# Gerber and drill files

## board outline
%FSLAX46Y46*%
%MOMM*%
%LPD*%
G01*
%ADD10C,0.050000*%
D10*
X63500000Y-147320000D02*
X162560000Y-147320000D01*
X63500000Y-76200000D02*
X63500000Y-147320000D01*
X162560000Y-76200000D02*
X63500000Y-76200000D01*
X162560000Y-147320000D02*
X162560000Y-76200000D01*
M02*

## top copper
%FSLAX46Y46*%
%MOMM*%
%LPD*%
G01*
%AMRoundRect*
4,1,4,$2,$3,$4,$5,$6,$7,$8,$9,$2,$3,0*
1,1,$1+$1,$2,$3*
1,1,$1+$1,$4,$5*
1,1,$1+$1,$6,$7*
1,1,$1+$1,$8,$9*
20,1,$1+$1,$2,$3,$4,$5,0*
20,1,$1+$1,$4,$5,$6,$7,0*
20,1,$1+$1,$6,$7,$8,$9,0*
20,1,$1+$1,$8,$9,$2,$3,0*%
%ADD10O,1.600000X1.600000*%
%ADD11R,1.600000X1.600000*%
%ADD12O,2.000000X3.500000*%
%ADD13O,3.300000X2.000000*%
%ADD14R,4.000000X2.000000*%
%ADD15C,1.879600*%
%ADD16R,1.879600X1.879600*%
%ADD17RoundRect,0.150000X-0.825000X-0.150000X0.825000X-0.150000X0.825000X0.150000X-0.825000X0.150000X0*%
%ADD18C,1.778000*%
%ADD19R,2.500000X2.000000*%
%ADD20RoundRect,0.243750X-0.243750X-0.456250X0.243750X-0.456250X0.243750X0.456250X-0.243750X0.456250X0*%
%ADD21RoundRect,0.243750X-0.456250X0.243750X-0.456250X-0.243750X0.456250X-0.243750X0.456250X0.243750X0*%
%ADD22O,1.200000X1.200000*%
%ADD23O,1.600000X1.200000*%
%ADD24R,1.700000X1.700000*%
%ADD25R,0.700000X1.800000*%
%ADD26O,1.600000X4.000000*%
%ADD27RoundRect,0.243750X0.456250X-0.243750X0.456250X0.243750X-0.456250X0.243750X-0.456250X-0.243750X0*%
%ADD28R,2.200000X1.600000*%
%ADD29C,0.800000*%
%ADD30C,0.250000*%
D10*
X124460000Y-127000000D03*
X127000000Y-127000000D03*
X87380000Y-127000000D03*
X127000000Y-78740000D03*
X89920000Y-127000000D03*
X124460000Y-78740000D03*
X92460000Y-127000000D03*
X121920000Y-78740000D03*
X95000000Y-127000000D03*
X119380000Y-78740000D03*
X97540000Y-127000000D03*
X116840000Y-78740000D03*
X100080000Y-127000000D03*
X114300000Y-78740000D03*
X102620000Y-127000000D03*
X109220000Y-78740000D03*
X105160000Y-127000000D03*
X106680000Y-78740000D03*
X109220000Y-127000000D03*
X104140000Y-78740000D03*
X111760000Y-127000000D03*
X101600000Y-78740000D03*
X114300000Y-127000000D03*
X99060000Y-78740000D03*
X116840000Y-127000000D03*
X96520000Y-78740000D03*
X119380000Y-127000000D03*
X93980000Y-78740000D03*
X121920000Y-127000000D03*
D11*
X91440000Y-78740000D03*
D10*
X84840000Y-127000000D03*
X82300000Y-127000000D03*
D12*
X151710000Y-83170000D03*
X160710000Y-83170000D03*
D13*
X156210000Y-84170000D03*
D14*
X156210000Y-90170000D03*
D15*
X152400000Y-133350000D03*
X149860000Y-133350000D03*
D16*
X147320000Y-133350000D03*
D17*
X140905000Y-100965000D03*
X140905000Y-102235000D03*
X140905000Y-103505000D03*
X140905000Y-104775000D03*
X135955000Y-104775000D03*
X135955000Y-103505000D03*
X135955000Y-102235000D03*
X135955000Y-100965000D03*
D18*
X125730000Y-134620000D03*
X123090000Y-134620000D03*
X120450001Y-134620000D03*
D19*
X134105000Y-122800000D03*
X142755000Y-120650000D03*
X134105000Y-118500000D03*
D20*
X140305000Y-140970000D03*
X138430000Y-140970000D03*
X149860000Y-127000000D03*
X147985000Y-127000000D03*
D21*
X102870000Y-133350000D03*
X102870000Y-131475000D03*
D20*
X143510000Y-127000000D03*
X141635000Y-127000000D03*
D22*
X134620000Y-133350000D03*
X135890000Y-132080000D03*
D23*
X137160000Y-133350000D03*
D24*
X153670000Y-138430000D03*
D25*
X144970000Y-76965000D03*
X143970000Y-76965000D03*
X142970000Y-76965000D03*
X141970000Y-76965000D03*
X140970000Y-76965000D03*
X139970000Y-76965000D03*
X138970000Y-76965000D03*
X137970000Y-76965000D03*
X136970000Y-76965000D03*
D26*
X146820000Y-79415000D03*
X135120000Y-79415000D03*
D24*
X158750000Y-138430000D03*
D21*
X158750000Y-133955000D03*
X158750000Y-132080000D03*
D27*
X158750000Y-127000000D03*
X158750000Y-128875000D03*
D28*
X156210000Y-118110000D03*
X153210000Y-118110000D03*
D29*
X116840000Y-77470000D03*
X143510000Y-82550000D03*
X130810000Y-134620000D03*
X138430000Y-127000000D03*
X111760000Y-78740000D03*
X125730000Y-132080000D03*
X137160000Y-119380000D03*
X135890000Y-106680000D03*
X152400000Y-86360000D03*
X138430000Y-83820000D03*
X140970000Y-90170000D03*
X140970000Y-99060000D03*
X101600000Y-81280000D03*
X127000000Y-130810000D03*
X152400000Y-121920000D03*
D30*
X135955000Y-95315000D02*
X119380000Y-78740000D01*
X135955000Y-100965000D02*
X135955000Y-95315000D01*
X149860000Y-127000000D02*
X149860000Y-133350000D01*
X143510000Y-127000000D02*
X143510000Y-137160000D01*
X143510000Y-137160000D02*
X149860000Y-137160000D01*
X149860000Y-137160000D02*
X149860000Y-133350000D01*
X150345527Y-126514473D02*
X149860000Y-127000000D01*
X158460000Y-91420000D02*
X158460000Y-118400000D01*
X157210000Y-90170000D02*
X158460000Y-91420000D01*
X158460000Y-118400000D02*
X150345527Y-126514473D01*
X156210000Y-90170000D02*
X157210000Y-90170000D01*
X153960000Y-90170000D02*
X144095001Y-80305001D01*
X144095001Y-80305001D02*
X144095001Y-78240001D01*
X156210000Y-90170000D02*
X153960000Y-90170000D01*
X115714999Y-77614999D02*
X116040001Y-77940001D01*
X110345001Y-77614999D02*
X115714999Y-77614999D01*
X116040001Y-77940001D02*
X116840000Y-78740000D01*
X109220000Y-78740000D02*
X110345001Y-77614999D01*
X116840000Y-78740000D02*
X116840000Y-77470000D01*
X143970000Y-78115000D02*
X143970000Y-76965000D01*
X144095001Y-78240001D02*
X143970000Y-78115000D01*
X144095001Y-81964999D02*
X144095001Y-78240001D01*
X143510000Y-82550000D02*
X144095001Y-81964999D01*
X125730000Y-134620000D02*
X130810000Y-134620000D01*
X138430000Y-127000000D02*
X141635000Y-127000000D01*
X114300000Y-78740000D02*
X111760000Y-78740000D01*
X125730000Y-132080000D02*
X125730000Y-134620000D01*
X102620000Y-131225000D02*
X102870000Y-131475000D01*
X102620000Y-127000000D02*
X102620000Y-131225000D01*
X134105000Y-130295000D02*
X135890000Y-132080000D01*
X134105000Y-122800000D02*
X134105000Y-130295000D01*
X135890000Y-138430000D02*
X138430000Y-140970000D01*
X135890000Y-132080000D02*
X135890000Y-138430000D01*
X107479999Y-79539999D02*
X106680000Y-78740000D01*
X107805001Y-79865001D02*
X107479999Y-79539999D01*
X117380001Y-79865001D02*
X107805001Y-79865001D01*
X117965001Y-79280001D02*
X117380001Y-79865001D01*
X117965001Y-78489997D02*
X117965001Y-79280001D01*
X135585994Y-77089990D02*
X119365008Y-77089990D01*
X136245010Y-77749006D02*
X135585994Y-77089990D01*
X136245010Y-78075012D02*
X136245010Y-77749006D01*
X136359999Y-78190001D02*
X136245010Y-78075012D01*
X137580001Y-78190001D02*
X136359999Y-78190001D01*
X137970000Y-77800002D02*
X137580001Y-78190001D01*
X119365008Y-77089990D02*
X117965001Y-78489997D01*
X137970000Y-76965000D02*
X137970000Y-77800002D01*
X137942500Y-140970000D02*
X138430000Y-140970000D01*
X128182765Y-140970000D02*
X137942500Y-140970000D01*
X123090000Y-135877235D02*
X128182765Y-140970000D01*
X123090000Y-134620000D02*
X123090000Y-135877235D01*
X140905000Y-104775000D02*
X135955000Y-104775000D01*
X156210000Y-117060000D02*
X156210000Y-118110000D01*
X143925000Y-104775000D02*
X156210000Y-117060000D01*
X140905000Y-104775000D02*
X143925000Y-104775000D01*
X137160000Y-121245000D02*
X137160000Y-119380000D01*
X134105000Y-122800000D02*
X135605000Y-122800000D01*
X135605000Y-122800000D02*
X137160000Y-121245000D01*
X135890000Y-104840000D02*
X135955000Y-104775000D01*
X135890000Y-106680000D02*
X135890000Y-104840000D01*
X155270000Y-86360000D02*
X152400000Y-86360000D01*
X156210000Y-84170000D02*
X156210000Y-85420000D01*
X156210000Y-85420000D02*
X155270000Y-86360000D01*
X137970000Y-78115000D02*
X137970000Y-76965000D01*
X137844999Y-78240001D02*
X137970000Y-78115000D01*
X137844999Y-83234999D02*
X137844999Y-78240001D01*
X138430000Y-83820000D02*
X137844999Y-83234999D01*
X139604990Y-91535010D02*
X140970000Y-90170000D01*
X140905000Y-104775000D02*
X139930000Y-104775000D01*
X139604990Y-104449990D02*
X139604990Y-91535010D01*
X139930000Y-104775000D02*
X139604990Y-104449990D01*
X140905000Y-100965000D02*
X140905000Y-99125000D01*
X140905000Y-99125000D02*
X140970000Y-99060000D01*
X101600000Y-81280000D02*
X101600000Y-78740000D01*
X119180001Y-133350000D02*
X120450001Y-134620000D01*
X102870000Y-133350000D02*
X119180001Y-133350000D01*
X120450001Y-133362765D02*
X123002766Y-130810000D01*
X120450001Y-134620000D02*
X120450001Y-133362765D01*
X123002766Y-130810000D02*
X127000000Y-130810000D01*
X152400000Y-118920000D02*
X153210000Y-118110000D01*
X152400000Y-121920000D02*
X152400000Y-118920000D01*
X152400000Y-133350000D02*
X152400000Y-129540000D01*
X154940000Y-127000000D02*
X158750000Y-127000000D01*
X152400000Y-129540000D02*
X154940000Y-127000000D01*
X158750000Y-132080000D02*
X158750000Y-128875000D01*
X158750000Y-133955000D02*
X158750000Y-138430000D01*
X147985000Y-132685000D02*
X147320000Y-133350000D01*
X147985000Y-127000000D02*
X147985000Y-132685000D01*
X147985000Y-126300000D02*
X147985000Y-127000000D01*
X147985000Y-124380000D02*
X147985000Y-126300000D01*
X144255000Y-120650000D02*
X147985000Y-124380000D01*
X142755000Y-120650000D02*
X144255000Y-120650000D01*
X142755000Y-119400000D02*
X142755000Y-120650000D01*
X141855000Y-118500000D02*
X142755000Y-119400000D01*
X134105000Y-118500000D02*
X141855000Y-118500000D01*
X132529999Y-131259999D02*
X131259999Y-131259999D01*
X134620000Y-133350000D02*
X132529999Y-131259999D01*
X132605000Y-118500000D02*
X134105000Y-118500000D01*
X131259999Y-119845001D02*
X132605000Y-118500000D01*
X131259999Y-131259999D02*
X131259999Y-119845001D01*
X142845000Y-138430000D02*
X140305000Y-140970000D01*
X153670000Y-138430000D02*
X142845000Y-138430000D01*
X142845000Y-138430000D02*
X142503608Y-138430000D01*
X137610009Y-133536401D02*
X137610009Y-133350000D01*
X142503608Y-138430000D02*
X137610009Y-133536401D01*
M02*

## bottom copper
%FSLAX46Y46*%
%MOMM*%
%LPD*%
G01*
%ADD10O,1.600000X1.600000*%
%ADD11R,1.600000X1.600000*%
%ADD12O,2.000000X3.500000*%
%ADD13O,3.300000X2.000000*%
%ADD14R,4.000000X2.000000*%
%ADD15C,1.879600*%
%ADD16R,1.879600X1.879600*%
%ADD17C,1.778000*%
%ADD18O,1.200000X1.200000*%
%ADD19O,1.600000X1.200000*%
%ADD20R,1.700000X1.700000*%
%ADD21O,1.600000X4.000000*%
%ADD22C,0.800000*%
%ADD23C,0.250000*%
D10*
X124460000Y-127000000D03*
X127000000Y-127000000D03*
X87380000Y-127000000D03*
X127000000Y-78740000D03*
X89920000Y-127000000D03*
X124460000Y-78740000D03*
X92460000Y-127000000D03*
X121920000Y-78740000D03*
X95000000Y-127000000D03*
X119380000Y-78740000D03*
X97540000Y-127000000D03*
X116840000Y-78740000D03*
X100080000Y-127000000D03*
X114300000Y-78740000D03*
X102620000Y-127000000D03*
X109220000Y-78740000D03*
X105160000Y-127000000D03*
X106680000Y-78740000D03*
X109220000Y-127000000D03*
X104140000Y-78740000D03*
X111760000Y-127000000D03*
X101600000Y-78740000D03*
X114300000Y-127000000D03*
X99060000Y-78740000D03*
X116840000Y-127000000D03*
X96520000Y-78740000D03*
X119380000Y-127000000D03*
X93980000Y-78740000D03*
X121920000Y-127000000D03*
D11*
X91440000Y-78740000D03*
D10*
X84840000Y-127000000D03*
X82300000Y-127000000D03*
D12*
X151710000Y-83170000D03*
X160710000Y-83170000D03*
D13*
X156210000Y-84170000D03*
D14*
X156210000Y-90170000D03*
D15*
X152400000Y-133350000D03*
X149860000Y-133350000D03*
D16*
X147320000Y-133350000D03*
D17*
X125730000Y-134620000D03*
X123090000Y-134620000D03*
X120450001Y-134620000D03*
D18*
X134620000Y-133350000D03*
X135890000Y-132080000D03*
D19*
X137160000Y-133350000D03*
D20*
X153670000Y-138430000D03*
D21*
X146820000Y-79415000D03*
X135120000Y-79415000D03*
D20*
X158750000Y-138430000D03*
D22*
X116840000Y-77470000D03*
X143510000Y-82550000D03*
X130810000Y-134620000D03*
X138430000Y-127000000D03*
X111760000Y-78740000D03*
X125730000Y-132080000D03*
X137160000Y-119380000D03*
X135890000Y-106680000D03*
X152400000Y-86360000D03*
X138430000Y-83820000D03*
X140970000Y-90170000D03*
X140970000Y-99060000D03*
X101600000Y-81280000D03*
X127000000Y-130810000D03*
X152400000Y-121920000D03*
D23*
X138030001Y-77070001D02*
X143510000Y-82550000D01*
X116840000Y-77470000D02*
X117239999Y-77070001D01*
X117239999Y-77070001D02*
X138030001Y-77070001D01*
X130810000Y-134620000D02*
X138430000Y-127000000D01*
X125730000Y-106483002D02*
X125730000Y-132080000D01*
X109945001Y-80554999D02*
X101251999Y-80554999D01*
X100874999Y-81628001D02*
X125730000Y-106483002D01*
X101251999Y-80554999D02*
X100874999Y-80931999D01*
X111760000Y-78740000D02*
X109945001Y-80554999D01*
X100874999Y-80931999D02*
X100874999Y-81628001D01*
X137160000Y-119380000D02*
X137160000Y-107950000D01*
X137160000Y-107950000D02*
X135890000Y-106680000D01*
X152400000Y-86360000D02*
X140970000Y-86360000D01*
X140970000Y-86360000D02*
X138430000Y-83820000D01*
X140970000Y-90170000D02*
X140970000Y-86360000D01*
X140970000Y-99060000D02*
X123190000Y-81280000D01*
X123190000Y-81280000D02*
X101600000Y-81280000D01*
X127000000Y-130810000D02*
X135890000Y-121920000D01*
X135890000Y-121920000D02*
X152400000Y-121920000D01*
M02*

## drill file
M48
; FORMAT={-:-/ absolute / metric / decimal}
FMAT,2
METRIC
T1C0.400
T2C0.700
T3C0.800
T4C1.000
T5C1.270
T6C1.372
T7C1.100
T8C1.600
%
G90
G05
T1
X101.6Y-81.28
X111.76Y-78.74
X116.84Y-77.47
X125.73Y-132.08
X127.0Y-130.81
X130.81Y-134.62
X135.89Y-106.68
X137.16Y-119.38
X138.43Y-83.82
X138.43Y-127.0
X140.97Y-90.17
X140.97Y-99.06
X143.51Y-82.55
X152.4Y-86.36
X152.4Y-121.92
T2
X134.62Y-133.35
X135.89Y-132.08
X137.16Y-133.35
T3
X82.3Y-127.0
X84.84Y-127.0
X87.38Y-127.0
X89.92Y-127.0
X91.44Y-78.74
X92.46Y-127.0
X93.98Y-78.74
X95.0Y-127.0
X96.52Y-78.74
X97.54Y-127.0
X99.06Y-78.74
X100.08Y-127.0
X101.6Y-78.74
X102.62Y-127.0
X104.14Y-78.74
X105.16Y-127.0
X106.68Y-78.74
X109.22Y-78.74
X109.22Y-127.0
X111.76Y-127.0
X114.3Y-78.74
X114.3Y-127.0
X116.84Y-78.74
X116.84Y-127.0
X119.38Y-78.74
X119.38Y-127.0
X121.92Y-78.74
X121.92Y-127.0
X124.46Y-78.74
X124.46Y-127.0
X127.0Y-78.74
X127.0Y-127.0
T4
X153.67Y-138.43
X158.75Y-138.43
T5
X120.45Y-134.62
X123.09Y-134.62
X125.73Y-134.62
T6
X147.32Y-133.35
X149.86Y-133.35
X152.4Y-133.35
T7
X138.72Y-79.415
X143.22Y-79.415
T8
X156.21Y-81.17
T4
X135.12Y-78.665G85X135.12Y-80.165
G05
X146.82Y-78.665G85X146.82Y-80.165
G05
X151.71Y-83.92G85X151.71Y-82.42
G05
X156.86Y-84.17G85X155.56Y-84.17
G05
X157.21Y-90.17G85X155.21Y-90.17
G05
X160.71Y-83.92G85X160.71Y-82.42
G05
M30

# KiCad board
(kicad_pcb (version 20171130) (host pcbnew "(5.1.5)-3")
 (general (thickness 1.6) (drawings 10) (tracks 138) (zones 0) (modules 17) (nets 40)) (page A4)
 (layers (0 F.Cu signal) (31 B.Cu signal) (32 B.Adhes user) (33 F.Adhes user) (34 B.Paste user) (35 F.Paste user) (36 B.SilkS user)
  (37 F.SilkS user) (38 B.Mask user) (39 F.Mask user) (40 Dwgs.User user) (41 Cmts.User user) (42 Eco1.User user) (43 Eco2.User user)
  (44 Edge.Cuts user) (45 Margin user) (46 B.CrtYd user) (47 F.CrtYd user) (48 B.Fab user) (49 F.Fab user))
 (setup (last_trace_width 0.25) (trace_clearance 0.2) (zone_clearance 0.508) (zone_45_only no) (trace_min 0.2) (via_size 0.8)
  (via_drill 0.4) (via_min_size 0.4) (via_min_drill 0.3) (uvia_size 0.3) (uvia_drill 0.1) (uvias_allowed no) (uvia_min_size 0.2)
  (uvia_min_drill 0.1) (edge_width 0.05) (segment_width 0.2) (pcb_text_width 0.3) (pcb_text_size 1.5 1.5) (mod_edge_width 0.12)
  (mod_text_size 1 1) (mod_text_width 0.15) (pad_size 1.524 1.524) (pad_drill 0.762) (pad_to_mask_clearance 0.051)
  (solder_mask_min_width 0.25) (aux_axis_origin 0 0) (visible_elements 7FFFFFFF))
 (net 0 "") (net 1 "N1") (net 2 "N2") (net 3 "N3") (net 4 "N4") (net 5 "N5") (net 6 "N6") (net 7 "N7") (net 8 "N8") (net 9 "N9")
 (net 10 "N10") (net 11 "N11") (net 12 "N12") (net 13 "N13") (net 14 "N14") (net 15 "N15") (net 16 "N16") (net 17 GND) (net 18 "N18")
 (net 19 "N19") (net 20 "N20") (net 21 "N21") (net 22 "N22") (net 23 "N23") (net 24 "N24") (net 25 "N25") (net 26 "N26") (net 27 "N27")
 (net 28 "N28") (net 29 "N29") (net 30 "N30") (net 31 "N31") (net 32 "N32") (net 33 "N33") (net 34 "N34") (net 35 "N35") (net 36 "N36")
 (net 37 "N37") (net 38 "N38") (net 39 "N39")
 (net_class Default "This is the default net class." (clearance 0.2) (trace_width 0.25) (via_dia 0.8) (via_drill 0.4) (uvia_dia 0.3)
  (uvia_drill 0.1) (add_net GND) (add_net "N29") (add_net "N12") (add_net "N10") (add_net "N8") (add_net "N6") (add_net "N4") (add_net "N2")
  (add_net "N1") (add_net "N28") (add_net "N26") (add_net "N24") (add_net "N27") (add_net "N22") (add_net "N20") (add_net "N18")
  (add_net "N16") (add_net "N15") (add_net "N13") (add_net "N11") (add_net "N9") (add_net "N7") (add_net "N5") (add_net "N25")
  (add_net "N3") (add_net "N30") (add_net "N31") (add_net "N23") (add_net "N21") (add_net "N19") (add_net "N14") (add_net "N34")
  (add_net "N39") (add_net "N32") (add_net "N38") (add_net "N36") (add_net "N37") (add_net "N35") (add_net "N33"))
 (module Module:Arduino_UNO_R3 (layer F.Cu) (at 91.44 78.74)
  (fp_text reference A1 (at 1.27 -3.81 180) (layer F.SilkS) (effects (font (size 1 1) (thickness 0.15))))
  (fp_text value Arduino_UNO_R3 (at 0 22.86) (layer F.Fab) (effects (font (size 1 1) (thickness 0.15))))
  (pad 16 thru_hole oval (at 33.02 48.26 90) (size 1.6 1.6) (drill 0.8) (layers *.Cu *.Mask) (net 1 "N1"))
  (pad 15 thru_hole oval (at 35.56 48.26 90) (size 1.6 1.6) (drill 0.8) (layers *.Cu *.Mask) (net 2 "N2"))
  (pad 30 thru_hole oval (at -4.06 48.26 90) (size 1.6 1.6) (drill 0.8) (layers *.Cu *.Mask) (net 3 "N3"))
  (pad 14 thru_hole oval (at 35.56 0 90) (size 1.6 1.6) (drill 0.8) (layers *.Cu *.Mask) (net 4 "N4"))
  (pad 29 thru_hole oval (at -1.52 48.26 90) (size 1.6 1.6) (drill 0.8) (layers *.Cu *.Mask) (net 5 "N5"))
  (pad 13 thru_hole oval (at 33.02 0 90) (size 1.6 1.6) (drill 0.8) (layers *.Cu *.Mask) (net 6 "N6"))
  (pad 28 thru_hole oval (at 1.02 48.26 90) (size 1.6 1.6) (drill 0.8) (layers *.Cu *.Mask) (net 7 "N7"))
  (pad 12 thru_hole oval (at 30.48 0 90) (size 1.6 1.6) (drill 0.8) (layers *.Cu *.Mask) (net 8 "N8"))
  (pad 27 thru_hole oval (at 3.56 48.26 90) (size 1.6 1.6) (drill 0.8) (layers *.Cu *.Mask) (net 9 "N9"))
  (pad 11 thru_hole oval (at 27.94 0 90) (size 1.6 1.6) (drill 0.8) (layers *.Cu *.Mask) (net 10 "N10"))
  (pad 26 thru_hole oval (at 6.1 48.26 90) (size 1.6 1.6) (drill 0.8) (layers *.Cu *.Mask) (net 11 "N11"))
  (pad 10 thru_hole oval (at 25.4 0 90) (size 1.6 1.6) (drill 0.8) (layers *.Cu *.Mask) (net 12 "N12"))
  (pad 25 thru_hole oval (at 8.64 48.26 90) (size 1.6 1.6) (drill 0.8) (layers *.Cu *.Mask) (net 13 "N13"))
  (pad 9 thru_hole oval (at 22.86 0 90) (size 1.6 1.6) (drill 0.8) (layers *.Cu *.Mask) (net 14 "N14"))
  (pad 24 thru_hole oval (at 11.18 48.26 90) (size 1.6 1.6) (drill 0.8) (layers *.Cu *.Mask) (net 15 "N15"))
  (pad 8 thru_hole oval (at 17.78 0 90) (size 1.6 1.6) (drill 0.8) (layers *.Cu *.Mask) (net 12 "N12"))
  (pad 23 thru_hole oval (at 13.72 48.26 90) (size 1.6 1.6) (drill 0.8) (layers *.Cu *.Mask) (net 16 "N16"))
  (pad 7 thru_hole oval (at 15.24 0 90) (size 1.6 1.6) (drill 0.8) (layers *.Cu *.Mask) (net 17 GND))
  (pad 22 thru_hole oval (at 17.78 48.26 90) (size 1.6 1.6) (drill 0.8) (layers *.Cu *.Mask) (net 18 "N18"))
  (pad 6 thru_hole oval (at 12.7 0 90) (size 1.6 1.6) (drill 0.8) (layers *.Cu *.Mask) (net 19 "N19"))
  (pad 21 thru_hole oval (at 20.32 48.26 90) (size 1.6 1.6) (drill 0.8) (layers *.Cu *.Mask) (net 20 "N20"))
  (pad 5 thru_hole oval (at 10.16 0 90) (size 1.6 1.6) (drill 0.8) (layers *.Cu *.Mask) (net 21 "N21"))
  (pad 20 thru_hole oval (at 22.86 48.26 90) (size 1.6 1.6) (drill 0.8) (layers *.Cu *.Mask) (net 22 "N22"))
  (pad 4 thru_hole oval (at 7.62 0 90) (size 1.6 1.6) (drill 0.8) (layers *.Cu *.Mask) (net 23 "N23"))
  (pad 19 thru_hole oval (at 25.4 48.26 90) (size 1.6 1.6) (drill 0.8) (layers *.Cu *.Mask) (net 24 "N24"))
  (pad 3 thru_hole oval (at 5.08 0 90) (size 1.6 1.6) (drill 0.8) (layers *.Cu *.Mask) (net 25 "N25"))
  (pad 18 thru_hole oval (at 27.94 48.26 90) (size 1.6 1.6) (drill 0.8) (layers *.Cu *.Mask) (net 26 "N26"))
  (pad 2 thru_hole oval (at 2.54 0 90) (size 1.6 1.6) (drill 0.8) (layers *.Cu *.Mask) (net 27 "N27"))
  (pad 17 thru_hole oval (at 30.48 48.26 90) (size 1.6 1.6) (drill 0.8) (layers *.Cu *.Mask) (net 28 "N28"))
  (pad 1 thru_hole rect (at 0 0 90) (size 1.6 1.6) (drill 0.8) (layers *.Cu *.Mask) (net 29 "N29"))
  (pad 31 thru_hole oval (at -6.6 48.26 90) (size 1.6 1.6) (drill 0.8) (layers *.Cu *.Mask) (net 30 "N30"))
  (pad 32 thru_hole oval (at -9.14 48.26 90) (size 1.6 1.6) (drill 0.8) (layers *.Cu *.Mask) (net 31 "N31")))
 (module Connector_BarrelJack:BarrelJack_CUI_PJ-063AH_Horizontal (layer F.Cu) (at 156.21 90.17 180)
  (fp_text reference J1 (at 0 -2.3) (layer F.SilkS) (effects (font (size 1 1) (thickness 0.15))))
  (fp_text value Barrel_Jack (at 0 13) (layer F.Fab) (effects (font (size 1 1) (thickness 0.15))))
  (pad "" np_thru_hole circle (at 0 9 180) (size 1.6 1.6) (drill 1.6) (layers *.Cu *.Mask))
  (pad MP thru_hole oval (at 4.5 7 180) (size 2 3.5) (drill oval 1 2.5) (layers *.Cu *.Mask))
  (pad MP thru_hole oval (at -4.5 7 180) (size 2 3.5) (drill oval 1 2.5) (layers *.Cu *.Mask))
  (pad 2 thru_hole oval (at 0 6 180) (size 3.3 2) (drill oval 2.3 1) (layers *.Cu *.Mask) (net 17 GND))
  (pad 1 thru_hole rect (at 0 0 180) (size 4 2) (drill oval 3 1) (layers *.Cu *.Mask) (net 12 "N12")))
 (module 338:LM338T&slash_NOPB (layer F.Cu) (at 147.32 133.35)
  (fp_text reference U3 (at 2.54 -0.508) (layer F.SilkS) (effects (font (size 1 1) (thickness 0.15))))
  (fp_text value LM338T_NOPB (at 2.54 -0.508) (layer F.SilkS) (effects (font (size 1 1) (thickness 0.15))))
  (pad 3 thru_hole circle (at 5.08 0) (size 1.8796 1.8796) (drill 1.3716) (layers *.Cu *.Mask) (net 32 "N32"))
  (pad 2 thru_hole circle (at 2.54 0) (size 1.8796 1.8796) (drill 1.3716) (layers *.Cu *.Mask) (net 12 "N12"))
  (pad 1 thru_hole rect (at 0 0) (size 1.8796 1.8796) (drill 1.3716) (layers *.Cu *.Mask) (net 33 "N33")))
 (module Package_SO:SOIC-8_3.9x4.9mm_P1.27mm (layer F.Cu) (at 138.43 102.87)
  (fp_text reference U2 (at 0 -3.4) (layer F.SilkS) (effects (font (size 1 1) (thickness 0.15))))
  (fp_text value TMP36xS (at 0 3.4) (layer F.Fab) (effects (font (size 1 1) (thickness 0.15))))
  (pad 8 smd roundrect (at 2.475 -1.905) (size 1.95 0.6) (layers F.Cu F.Paste F.Mask) (roundrect_rratio 0.25) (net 21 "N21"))
  (pad 7 smd roundrect (at 2.475 -0.635) (size 1.95 0.6) (layers F.Cu F.Paste F.Mask) (roundrect_rratio 0.25))
  (pad 6 smd roundrect (at 2.475 0.635) (size 1.95 0.6) (layers F.Cu F.Paste F.Mask) (roundrect_rratio 0.25))
  (pad 5 smd roundrect (at 2.475 1.905) (size 1.95 0.6) (layers F.Cu F.Paste F.Mask) (roundrect_rratio 0.25) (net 17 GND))
  (pad 4 smd roundrect (at -2.475 1.905) (size 1.95 0.6) (layers F.Cu F.Paste F.Mask) (roundrect_rratio 0.25) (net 17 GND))
  (pad 3 smd roundrect (at -2.475 0.635) (size 1.95 0.6) (layers F.Cu F.Paste F.Mask) (roundrect_rratio 0.25))
  (pad 2 smd roundrect (at -2.475 -0.635) (size 1.95 0.6) (layers F.Cu F.Paste F.Mask) (roundrect_rratio 0.25))
  (pad 1 smd roundrect (at -2.475 -1.905) (size 1.95 0.6) (layers F.Cu F.Paste F.Mask) (roundrect_rratio 0.25) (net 10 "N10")))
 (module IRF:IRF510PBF (layer F.Cu) (at 125.73 134.62)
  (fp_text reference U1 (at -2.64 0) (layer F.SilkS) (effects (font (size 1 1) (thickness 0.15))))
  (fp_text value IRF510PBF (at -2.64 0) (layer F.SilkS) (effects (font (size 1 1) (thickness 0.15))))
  (pad 3 thru_hole circle (at 0 0) (size 1.778 1.778) (drill 1.27) (layers *.Cu *.Mask) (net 14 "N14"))
  (pad 2 thru_hole circle (at -2.64 0) (size 1.778 1.778) (drill 1.27) (layers *.Cu *.Mask) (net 17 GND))
  (pad 1 thru_hole circle (at -5.279999 0) (size 1.778 1.778) (drill 1.27) (layers *.Cu *.Mask) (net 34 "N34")))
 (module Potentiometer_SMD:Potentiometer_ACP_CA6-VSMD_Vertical (layer F.Cu) (at 138.43 120.65)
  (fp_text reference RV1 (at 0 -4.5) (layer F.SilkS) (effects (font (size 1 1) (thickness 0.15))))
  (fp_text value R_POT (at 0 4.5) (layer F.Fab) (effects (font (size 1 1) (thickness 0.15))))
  (pad 1 smd rect (at -4.325 2.15) (size 2.5 2) (layers F.Cu F.Paste F.Mask) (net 17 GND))
  (pad 2 smd rect (at 4.325 0) (size 2.5 2) (layers F.Cu F.Paste F.Mask) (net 33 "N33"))
  (pad 3 smd rect (at -4.325 -2.15) (size 2.5 2) (layers F.Cu F.Paste F.Mask) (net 33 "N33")))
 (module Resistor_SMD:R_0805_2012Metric (layer F.Cu) (at 139.3675 140.97)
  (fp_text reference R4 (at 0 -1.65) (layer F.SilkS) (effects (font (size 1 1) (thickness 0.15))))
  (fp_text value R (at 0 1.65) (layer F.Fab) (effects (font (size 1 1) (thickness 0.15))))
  (pad 2 smd roundrect (at 0.9375 0) (size 0.975 1.4) (layers F.Cu F.Paste F.Mask) (roundrect_rratio 0.25) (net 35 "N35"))
  (pad 1 smd roundrect (at -0.9375 0) (size 0.975 1.4) (layers F.Cu F.Paste F.Mask) (roundrect_rratio 0.25) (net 17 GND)))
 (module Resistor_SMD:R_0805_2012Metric (layer F.Cu) (at 148.9225 127)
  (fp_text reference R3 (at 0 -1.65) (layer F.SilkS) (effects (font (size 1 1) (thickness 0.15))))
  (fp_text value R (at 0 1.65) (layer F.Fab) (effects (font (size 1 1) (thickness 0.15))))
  (pad 2 smd roundrect (at 0.9375 0) (size 0.975 1.4) (layers F.Cu F.Paste F.Mask) (roundrect_rratio 0.25) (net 12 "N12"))
  (pad 1 smd roundrect (at -0.9375 0) (size 0.975 1.4) (layers F.Cu F.Paste F.Mask) (roundrect_rratio 0.25) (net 33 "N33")))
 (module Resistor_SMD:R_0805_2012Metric (layer F.Cu) (at 102.87 132.4125 270)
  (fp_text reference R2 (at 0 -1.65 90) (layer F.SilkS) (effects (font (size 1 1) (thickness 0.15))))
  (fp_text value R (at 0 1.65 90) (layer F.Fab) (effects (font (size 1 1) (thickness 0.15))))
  (pad 2 smd roundrect (at 0.9375 0 270) (size 0.975 1.4) (layers F.Cu F.Paste F.Mask) (roundrect_rratio 0.25) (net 34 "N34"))
  (pad 1 smd roundrect (at -0.9375 0 270) (size 0.975 1.4) (layers F.Cu F.Paste F.Mask) (roundrect_rratio 0.25) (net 15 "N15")))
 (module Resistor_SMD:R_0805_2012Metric (layer F.Cu) (at 142.5725 127)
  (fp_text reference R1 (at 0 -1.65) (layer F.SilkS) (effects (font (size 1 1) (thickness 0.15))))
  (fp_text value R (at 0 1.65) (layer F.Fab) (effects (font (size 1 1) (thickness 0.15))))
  (pad 2 smd roundrect (at 0.9375 0) (size 0.975 1.4) (layers F.Cu F.Paste F.Mask) (roundrect_rratio 0.25) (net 12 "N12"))
  (pad 1 smd roundrect (at -0.9375 0) (size 0.975 1.4) (layers F.Cu F.Paste F.Mask) (roundrect_rratio 0.25) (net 14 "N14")))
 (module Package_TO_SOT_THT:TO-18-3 (layer F.Cu) (at 137.16 133.35 180)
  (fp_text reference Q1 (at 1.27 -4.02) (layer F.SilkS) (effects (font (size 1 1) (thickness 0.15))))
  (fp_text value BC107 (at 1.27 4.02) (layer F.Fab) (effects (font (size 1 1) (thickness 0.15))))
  (pad 3 thru_hole oval (at 2.54 0 180) (size 1.2 1.2) (drill 0.7) (layers *.Cu *.Mask) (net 33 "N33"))
  (pad 2 thru_hole oval (at 1.27 1.27 180) (size 1.2 1.2) (drill 0.7) (layers *.Cu *.Mask) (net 17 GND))
  (pad 1 thru_hole oval (at 0 0 180) (size 1.6 1.2) (drill 0.7) (layers *.Cu *.Mask) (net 35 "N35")))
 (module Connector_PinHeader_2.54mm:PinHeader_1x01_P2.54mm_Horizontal (layer F.Cu) (at 153.67 138.43 270)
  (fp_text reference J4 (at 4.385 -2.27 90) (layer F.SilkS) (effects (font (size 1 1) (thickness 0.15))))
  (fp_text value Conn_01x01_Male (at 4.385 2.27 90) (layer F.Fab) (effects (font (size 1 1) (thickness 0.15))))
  (pad 1 thru_hole rect (at 0 0 270) (size 1.7 1.7) (drill 1) (layers *.Cu *.Mask) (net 35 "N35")))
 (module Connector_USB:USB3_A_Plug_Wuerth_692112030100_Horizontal (layer F.Cu) (at 140.97 78.74 270)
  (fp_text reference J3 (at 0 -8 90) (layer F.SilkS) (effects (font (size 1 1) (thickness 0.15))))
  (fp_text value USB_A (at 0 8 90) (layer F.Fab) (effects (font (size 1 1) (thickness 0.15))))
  (pad "" np_thru_hole circle (at 0.675 -2.25) (size 1.1 1.1) (drill 1.1) (layers *.Cu *.Mask))
  (pad "" np_thru_hole circle (at 0.675 2.25) (size 1.1 1.1) (drill 1.1) (layers *.Cu *.Mask))
  (pad 9 smd rect (at -1.775 -4 270) (size 1.8 0.7) (layers F.Cu F.Paste F.Mask))
  (pad 1 smd rect (at -1.775 -3) (size 0.7 1.8) (layers F.Cu F.Paste F.Mask) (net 12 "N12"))
  (pad 8 smd rect (at -1.775 -2) (size 0.7 1.8) (layers F.Cu F.Paste F.Mask))
  (pad 2 smd rect (at -1.775 -1) (size 0.7 1.8) (layers F.Cu F.Paste F.Mask) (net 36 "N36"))
  (pad 7 smd rect (at -1.775 0) (size 0.7 1.8) (layers F.Cu F.Paste F.Mask))
  (pad 3 smd rect (at -1.775 1) (size 0.7 1.8) (layers F.Cu F.Paste F.Mask) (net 36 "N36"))
  (pad 6 smd rect (at -1.775 2) (size 0.7 1.8) (layers F.Cu F.Paste F.Mask))
  (pad 4 smd rect (at -1.775 3) (size 0.7 1.8) (layers F.Cu F.Paste F.Mask) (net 17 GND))
  (pad 5 smd rect (at -1.775 4) (size 0.7 1.8) (layers F.Cu F.Paste F.Mask) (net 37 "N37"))
  (pad 10 thru_hole oval (at 0.675 -5.85) (size 1.6 4) (drill oval 1 2.5) (layers *.Cu *.Mask))
  (pad 10 thru_hole oval (at 0.675 5.85) (size 1.6 4) (drill oval 1 2.5) (layers *.Cu *.Mask)))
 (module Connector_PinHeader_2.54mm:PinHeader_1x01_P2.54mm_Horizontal (layer F.Cu) (at 158.75 138.43 270)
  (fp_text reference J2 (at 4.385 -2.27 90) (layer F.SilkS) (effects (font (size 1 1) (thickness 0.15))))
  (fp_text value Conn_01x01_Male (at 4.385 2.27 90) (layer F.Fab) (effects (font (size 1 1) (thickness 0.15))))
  (pad 1 thru_hole rect (at 0 0 270) (size 1.7 1.7) (drill 1) (layers *.Cu *.Mask) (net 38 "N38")))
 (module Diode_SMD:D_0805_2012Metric (layer F.Cu) (at 158.75 133.0175 270)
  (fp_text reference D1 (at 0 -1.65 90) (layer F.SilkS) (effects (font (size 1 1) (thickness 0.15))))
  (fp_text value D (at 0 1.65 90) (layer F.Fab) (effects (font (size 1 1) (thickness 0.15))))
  (pad 2 smd roundrect (at 0.9375 0 270) (size 0.975 1.4) (layers F.Cu F.Paste F.Mask) (roundrect_rratio 0.25) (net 38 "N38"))
  (pad 1 smd roundrect (at -0.9375 0 270) (size 0.975 1.4) (layers F.Cu F.Paste F.Mask) (roundrect_rratio 0.25) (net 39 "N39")))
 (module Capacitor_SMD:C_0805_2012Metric (layer F.Cu) (at 158.75 127.9375 90)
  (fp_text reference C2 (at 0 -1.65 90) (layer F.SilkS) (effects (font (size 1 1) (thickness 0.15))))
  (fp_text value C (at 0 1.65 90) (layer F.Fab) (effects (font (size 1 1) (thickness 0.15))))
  (pad 2 smd roundrect (at 0.9375 0 90) (size 0.975 1.4) (layers F.Cu F.Paste F.Mask) (roundrect_rratio 0.25) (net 32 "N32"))
  (pad 1 smd roundrect (at -0.9375 0 90) (size 0.975 1.4) (layers F.Cu F.Paste F.Mask) (roundrect_rratio 0.25) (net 39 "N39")))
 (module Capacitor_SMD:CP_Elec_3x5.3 (layer F.Cu) (at 154.71 118.11)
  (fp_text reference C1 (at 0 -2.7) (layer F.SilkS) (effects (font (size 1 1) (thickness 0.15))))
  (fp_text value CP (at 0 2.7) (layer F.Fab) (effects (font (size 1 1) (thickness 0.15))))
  (pad 2 smd rect (at 1.5 0) (size 2.2 1.6) (layers F.Cu F.Paste F.Mask) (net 17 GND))
  (pad 1 smd rect (at -1.5 0) (size 2.2 1.6) (layers F.Cu F.Paste F.Mask) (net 34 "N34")))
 (gr_line (start 63.5 147.32) (end 162.56 147.32) (layer Edge.Cuts) (width 0.05))
 (gr_line (start 63.5 76.2) (end 63.5 147.32) (layer Edge.Cuts) (width 0.05))
 (gr_line (start 162.56 76.2) (end 63.5 76.2) (layer Edge.Cuts) (width 0.05))
 (gr_line (start 162.56 147.32) (end 162.56 76.2) (layer Edge.Cuts) (width 0.05))
 (segment (start 135.955 95.315) (end 119.38 78.74) (width 0.25) (layer F.Cu) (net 10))
 (segment (start 135.955 100.965) (end 135.955 95.315) (width 0.25) (layer F.Cu) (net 10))
 (segment (start 149.86 127) (end 149.86 133.35) (width 0.25) (layer F.Cu) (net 12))
 (segment (start 143.51 127) (end 143.51 137.16) (width 0.25) (layer F.Cu) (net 12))
 (segment (start 143.51 137.16) (end 149.86 137.16) (width 0.25) (layer F.Cu) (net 12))
 (segment (start 149.86 137.16) (end 149.86 133.35) (width 0.25) (layer F.Cu) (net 12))
 (segment (start 150.345527 126.514473) (end 149.86 127) (width 0.25) (layer F.Cu) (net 12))
 (segment (start 158.46 91.42) (end 158.46 118.4) (width 0.25) (layer F.Cu) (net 12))
 (segment (start 157.21 90.17) (end 158.46 91.42) (width 0.25) (layer F.Cu) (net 12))
 (segment (start 158.46 118.4) (end 150.345527 126.514473) (width 0.25) (layer F.Cu) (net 12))
 (segment (start 156.21 90.17) (end 157.21 90.17) (width 0.25) (layer F.Cu) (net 12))
 (segment (start 153.96 90.17) (end 144.095001 80.305001) (width 0.25) (layer F.Cu) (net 12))
 (segment (start 144.095001 80.305001) (end 144.095001 78.240001) (width 0.25) (layer F.Cu) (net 12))
 (segment (start 156.21 90.17) (end 153.96 90.17) (width 0.25) (layer F.Cu) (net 12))
 (segment (start 115.714999 77.614999) (end 116.040001 77.940001) (width 0.25) (layer F.Cu) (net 12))
 (segment (start 110.345001 77.614999) (end 115.714999 77.614999) (width 0.25) (layer F.Cu) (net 12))
 (segment (start 116.040001 77.940001) (end 116.84 78.74) (width 0.25) (layer F.Cu) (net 12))
 (segment (start 109.22 78.74) (end 110.345001 77.614999) (width 0.25) (layer F.Cu) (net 12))
 (via (at 116.84 77.47) (size 0.8) (drill 0.4) (layers F.Cu B.Cu) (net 12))
 (segment (start 116.84 78.74) (end 116.84 77.47) (width 0.25) (layer F.Cu) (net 12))
 (via (at 143.51 82.55) (size 0.8) (drill 0.4) (layers F.Cu B.Cu) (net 12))
 (segment (start 138.030001 77.070001) (end 143.51 82.55) (width 0.25) (layer B.Cu) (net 12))
 (segment (start 116.84 77.47) (end 117.239999 77.070001) (width 0.25) (layer B.Cu) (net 12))
 (segment (start 117.239999 77.070001) (end 138.030001 77.070001) (width 0.25) (layer B.Cu) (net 12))
 (segment (start 143.97 78.115) (end 143.97 76.965) (width 0.25) (layer F.Cu) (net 12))
 (segment (start 144.095001 78.240001) (end 143.97 78.115) (width 0.25) (layer F.Cu) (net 12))
 (segment (start 144.095001 81.964999) (end 144.095001 78.240001) (width 0.25) (layer F.Cu) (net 12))
 (segment (start 143.51 82.55) (end 144.095001 81.964999) (width 0.25) (layer F.Cu) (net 12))
 (via (at 130.81 134.62) (size 0.8) (drill 0.4) (layers F.Cu B.Cu) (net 14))
 (segment (start 125.73 134.62) (end 130.81 134.62) (width 0.25) (layer F.Cu) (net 14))
 (via (at 138.43 127) (size 0.8) (drill 0.4) (layers F.Cu B.Cu) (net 14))
 (segment (start 130.81 134.62) (end 138.43 127) (width 0.25) (layer B.Cu) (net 14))
 (segment (start 138.43 127) (end 141.635 127) (width 0.25) (layer F.Cu) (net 14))
 (via (at 111.76 78.74) (size 0.8) (drill 0.4) (layers F.Cu B.Cu) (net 14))
 (segment (start 114.3 78.74) (end 111.76 78.74) (width 0.25) (layer F.Cu) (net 14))
 (via (at 125.73 132.08) (size 0.8) (drill 0.4) (layers F.Cu B.Cu) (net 14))
 (segment (start 125.73 106.483002) (end 125.73 132.08) (width 0.25) (layer B.Cu) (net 14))
 (segment (start 109.945001 80.554999) (end 101.251999 80.554999) (width 0.25) (layer B.Cu) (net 14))
 (segment (start 100.874999 81.628001) (end 125.73 106.483002) (width 0.25) (layer B.Cu) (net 14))
 (segment (start 101.251999 80.554999) (end 100.874999 80.931999) (width 0.25) (layer B.Cu) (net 14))
 (segment (start 111.76 78.74) (end 109.945001 80.554999) (width 0.25) (layer B.Cu) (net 14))
 (segment (start 100.874999 80.931999) (end 100.874999 81.628001) (width 0.25) (layer B.Cu) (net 14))
 (segment (start 125.73 132.08) (end 125.73 134.62) (width 0.25) (layer F.Cu) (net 14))
 (segment (start 102.62 131.225) (end 102.87 131.475) (width 0.25) (layer F.Cu) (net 15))
 (segment (start 102.62 127) (end 102.62 131.225) (width 0.25) (layer F.Cu) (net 15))
 (segment (start 134.105 130.295) (end 135.89 132.08) (width 0.25) (layer F.Cu) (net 17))
 (segment (start 134.105 122.8) (end 134.105 130.295) (width 0.25) (layer F.Cu) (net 17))
 (segment (start 135.89 138.43) (end 138.43 140.97) (width 0.25) (layer F.Cu) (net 17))
 (segment (start 135.89 132.08) (end 135.89 138.43) (width 0.25) (layer F.Cu) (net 17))
 (segment (start 107.479999 79.539999) (end 106.68 78.74) (width 0.25) (layer F.Cu) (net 17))
 (segment (start 107.805001 79.865001) (end 107.479999 79.539999) (width 0.25) (layer F.Cu) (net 17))
 (segment (start 117.380001 79.865001) (end 107.805001 79.865001) (width 0.25) (layer F.Cu) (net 17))
 (segment (start 117.965001 79.280001) (end 117.380001 79.865001) (width 0.25) (layer F.Cu) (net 17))
 (segment (start 117.965001 78.489997) (end 117.965001 79.280001) (width 0.25) (layer F.Cu) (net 17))
 (segment (start 135.585994 77.08999) (end 119.365008 77.08999) (width 0.25) (layer F.Cu) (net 17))
 (segment (start 136.24501 77.749006) (end 135.585994 77.08999) (width 0.25) (layer F.Cu) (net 17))
 (segment (start 136.24501 78.075012) (end 136.24501 77.749006) (width 0.25) (layer F.Cu) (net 17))
 (segment (start 136.359999 78.190001) (end 136.24501 78.075012) (width 0.25) (layer F.Cu) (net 17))
 (segment (start 137.580001 78.190001) (end 136.359999 78.190001) (width 0.25) (layer F.Cu) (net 17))
 (segment (start 137.97 77.800002) (end 137.580001 78.190001) (width 0.25) (layer F.Cu) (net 17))
 (segment (start 119.365008 77.08999) (end 117.965001 78.489997) (width 0.25) (layer F.Cu) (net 17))
 (segment (start 137.97 76.965) (end 137.97 77.800002) (width 0.25) (layer F.Cu) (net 17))
 (segment (start 137.9425 140.97) (end 138.43 140.97) (width 0.25) (layer F.Cu) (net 17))
 (segment (start 128.182765 140.97) (end 137.9425 140.97) (width 0.25) (layer F.Cu) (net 17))
 (segment (start 123.09 135.877235) (end 128.182765 140.97) (width 0.25) (layer F.Cu) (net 17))
 (segment (start 123.09 134.62) (end 123.09 135.877235) (width 0.25) (layer F.Cu) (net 17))
 (segment (start 140.905 104.775) (end 135.955 104.775) (width 0.25) (layer F.Cu) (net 17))
 (segment (start 156.21 117.06) (end 156.21 118.11) (width 0.25) (layer F.Cu) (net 17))
 (segment (start 143.925 104.775) (end 156.21 117.06) (width 0.25) (layer F.Cu) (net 17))
 (segment (start 140.905 104.775) (end 143.925 104.775) (width 0.25) (layer F.Cu) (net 17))
 (via (at 137.16 119.38) (size 0.8) (drill 0.4) (layers F.Cu B.Cu) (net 17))
 (segment (start 137.16 121.245) (end 137.16 119.38) (width 0.25) (layer F.Cu) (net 17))
 (segment (start 134.105 122.8) (end 135.605 122.8) (width 0.25) (layer F.Cu) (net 17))
 (segment (start 135.605 122.8) (end 137.16 121.245) (width 0.25) (layer F.Cu) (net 17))
 (segment (start 137.16 119.38) (end 137.16 107.95) (width 0.25) (layer B.Cu) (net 17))
 (via (at 135.89 106.68) (size 0.8) (drill 0.4) (layers F.Cu B.Cu) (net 17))
 (segment (start 137.16 107.95) (end 135.89 106.68) (width 0.25) (layer B.Cu) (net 17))
 (segment (start 135.89 104.84) (end 135.955 104.775) (width 0.25) (layer F.Cu) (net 17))
 (segment (start 135.89 106.68) (end 135.89 104.84) (width 0.25) (layer F.Cu) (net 17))
 (via (at 152.4 86.36) (size 0.8) (drill 0.4) (layers F.Cu B.Cu) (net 17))
 (segment (start 155.27 86.36) (end 152.4 86.36) (width 0.25) (layer F.Cu) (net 17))
 (segment (start 156.21 84.17) (end 156.21 85.42) (width 0.25) (layer F.Cu) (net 17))
 (segment (start 156.21 85.42) (end 155.27 86.36) (width 0.25) (layer F.Cu) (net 17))
 (via (at 138.43 83.82) (size 0.8) (drill 0.4) (layers F.Cu B.Cu) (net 17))
 (segment (start 152.4 86.36) (end 140.97 86.36) (width 0.25) (layer B.Cu) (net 17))
 (segment (start 140.97 86.36) (end 138.43 83.82) (width 0.25) (layer B.Cu) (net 17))
 (segment (start 137.97 78.115) (end 137.97 76.965) (width 0.25) (layer F.Cu) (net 17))
 (segment (start 137.844999 78.240001) (end 137.97 78.115) (width 0.25) (layer F.Cu) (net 17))
 (segment (start 137.844999 83.234999) (end 137.844999 78.240001) (width 0.25) (layer F.Cu) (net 17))
 (segment (start 138.43 83.82) (end 137.844999 83.234999) (width 0.25) (layer F.Cu) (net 17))
 (via (at 140.97 90.17) (size 0.8) (drill 0.4) (layers F.Cu B.Cu) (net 17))
 (segment (start 139.60499 91.53501) (end 140.97 90.17) (width 0.25) (layer F.Cu) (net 17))
 (segment (start 140.905 104.775) (end 139.93 104.775) (width 0.25) (layer F.Cu) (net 17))
 (segment (start 139.60499 104.44999) (end 139.60499 91.53501) (width 0.25) (layer F.Cu) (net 17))
 (segment (start 139.93 104.775) (end 139.60499 104.44999) (width 0.25) (layer F.Cu) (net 17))
 (segment (start 140.97 90.17) (end 140.97 86.36) (width 0.25) (layer B.Cu) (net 17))
 (via (at 140.97 99.06) (size 0.8) (drill 0.4) (layers F.Cu B.Cu) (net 21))
 (segment (start 140.905 100.965) (end 140.905 99.125) (width 0.25) (layer F.Cu) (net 21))
 (segment (start 140.905 99.125) (end 140.97 99.06) (width 0.25) (layer F.Cu) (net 21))
 (via (at 101.6 81.28) (size 0.8) (drill 0.4) (layers F.Cu B.Cu) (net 21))
 (segment (start 140.97 99.06) (end 123.19 81.28) (width 0.25) (layer B.Cu) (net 21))
 (segment (start 123.19 81.28) (end 101.6 81.28) (width 0.25) (layer B.Cu) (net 21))
 (segment (start 101.6 81.28) (end 101.6 78.74) (width 0.25) (layer F.Cu) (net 21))
 (segment (start 119.180001 133.35) (end 120.450001 134.62) (width 0.25) (layer F.Cu) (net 34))
 (segment (start 102.87 133.35) (end 119.180001 133.35) (width 0.25) (layer F.Cu) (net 34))
 (segment (start 120.450001 133.362765) (end 123.002766 130.81) (width 0.25) (layer F.Cu) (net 34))
 (segment (start 120.450001 134.62) (end 120.450001 133.362765) (width 0.25) (layer F.Cu) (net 34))
 (via (at 127 130.81) (size 0.8) (drill 0.4) (layers F.Cu B.Cu) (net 34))
 (segment (start 123.002766 130.81) (end 127 130.81) (width 0.25) (layer F.Cu) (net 34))
 (via (at 152.4 121.92) (size 0.8) (drill 0.4) (layers F.Cu B.Cu) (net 34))
 (segment (start 127 130.81) (end 135.89 121.92) (width 0.25) (layer B.Cu) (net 34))
 (segment (start 135.89 121.92) (end 152.4 121.92) (width 0.25) (layer B.Cu) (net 34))
 (segment (start 152.4 118.92) (end 153.21 118.11) (width 0.25) (layer F.Cu) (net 34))
 (segment (start 152.4 121.92) (end 152.4 118.92) (width 0.25) (layer F.Cu) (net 34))
 (segment (start 152.4 133.35) (end 152.4 129.54) (width 0.25) (layer F.Cu) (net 32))
 (segment (start 154.94 127) (end 158.75 127) (width 0.25) (layer F.Cu) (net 32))
 (segment (start 152.4 129.54) (end 154.94 127) (width 0.25) (layer F.Cu) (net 32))
 (segment (start 158.75 132.08) (end 158.75 128.875) (width 0.25) (layer F.Cu) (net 39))
 (segment (start 158.75 133.955) (end 158.75 138.43) (width 0.25) (layer F.Cu) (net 38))
 (segment (start 147.985 132.685) (end 147.32 133.35) (width 0.25) (layer F.Cu) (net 33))
 (segment (start 147.985 127) (end 147.985 132.685) (width 0.25) (layer F.Cu) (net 33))
 (segment (start 147.985 126.3) (end 147.985 127) (width 0.25) (layer F.Cu) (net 33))
 (segment (start 147.985 124.38) (end 147.985 126.3) (width 0.25) (layer F.Cu) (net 33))
 (segment (start 144.255 120.65) (end 147.985 124.38) (width 0.25) (layer F.Cu) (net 33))
 (segment (start 142.755 120.65) (end 144.255 120.65) (width 0.25) (layer F.Cu) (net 33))
 (segment (start 142.755 119.4) (end 142.755 120.65) (width 0.25) (layer F.Cu) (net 33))
 (segment (start 141.855 118.5) (end 142.755 119.4) (width 0.25) (layer F.Cu) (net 33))
 (segment (start 134.105 118.5) (end 141.855 118.5) (width 0.25) (layer F.Cu) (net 33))
 (segment (start 132.529999 131.259999) (end 131.259999 131.259999) (width 0.25) (layer F.Cu) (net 33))
 (segment (start 134.62 133.35) (end 132.529999 131.259999) (width 0.25) (layer F.Cu) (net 33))
 (segment (start 132.605 118.5) (end 134.105 118.5) (width 0.25) (layer F.Cu) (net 33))
 (segment (start 131.259999 119.845001) (end 132.605 118.5) (width 0.25) (layer F.Cu) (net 33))
 (segment (start 131.259999 131.259999) (end 131.259999 119.845001) (width 0.25) (layer F.Cu) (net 33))
 (segment (start 142.845 138.43) (end 140.305 140.97) (width 0.25) (layer F.Cu) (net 35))
 (segment (start 153.67 138.43) (end 142.845 138.43) (width 0.25) (layer F.Cu) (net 35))
 (segment (start 142.845 138.43) (end 142.503608 138.43) (width 0.25) (layer F.Cu) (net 35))
 (segment (start 137.610009 133.536401) (end 137.610009 133.35) (width 0.25) (layer F.Cu) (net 35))
 (segment (start 142.503608 138.43) (end 137.610009 133.536401) (width 0.25) (layer F.Cu) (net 35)))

